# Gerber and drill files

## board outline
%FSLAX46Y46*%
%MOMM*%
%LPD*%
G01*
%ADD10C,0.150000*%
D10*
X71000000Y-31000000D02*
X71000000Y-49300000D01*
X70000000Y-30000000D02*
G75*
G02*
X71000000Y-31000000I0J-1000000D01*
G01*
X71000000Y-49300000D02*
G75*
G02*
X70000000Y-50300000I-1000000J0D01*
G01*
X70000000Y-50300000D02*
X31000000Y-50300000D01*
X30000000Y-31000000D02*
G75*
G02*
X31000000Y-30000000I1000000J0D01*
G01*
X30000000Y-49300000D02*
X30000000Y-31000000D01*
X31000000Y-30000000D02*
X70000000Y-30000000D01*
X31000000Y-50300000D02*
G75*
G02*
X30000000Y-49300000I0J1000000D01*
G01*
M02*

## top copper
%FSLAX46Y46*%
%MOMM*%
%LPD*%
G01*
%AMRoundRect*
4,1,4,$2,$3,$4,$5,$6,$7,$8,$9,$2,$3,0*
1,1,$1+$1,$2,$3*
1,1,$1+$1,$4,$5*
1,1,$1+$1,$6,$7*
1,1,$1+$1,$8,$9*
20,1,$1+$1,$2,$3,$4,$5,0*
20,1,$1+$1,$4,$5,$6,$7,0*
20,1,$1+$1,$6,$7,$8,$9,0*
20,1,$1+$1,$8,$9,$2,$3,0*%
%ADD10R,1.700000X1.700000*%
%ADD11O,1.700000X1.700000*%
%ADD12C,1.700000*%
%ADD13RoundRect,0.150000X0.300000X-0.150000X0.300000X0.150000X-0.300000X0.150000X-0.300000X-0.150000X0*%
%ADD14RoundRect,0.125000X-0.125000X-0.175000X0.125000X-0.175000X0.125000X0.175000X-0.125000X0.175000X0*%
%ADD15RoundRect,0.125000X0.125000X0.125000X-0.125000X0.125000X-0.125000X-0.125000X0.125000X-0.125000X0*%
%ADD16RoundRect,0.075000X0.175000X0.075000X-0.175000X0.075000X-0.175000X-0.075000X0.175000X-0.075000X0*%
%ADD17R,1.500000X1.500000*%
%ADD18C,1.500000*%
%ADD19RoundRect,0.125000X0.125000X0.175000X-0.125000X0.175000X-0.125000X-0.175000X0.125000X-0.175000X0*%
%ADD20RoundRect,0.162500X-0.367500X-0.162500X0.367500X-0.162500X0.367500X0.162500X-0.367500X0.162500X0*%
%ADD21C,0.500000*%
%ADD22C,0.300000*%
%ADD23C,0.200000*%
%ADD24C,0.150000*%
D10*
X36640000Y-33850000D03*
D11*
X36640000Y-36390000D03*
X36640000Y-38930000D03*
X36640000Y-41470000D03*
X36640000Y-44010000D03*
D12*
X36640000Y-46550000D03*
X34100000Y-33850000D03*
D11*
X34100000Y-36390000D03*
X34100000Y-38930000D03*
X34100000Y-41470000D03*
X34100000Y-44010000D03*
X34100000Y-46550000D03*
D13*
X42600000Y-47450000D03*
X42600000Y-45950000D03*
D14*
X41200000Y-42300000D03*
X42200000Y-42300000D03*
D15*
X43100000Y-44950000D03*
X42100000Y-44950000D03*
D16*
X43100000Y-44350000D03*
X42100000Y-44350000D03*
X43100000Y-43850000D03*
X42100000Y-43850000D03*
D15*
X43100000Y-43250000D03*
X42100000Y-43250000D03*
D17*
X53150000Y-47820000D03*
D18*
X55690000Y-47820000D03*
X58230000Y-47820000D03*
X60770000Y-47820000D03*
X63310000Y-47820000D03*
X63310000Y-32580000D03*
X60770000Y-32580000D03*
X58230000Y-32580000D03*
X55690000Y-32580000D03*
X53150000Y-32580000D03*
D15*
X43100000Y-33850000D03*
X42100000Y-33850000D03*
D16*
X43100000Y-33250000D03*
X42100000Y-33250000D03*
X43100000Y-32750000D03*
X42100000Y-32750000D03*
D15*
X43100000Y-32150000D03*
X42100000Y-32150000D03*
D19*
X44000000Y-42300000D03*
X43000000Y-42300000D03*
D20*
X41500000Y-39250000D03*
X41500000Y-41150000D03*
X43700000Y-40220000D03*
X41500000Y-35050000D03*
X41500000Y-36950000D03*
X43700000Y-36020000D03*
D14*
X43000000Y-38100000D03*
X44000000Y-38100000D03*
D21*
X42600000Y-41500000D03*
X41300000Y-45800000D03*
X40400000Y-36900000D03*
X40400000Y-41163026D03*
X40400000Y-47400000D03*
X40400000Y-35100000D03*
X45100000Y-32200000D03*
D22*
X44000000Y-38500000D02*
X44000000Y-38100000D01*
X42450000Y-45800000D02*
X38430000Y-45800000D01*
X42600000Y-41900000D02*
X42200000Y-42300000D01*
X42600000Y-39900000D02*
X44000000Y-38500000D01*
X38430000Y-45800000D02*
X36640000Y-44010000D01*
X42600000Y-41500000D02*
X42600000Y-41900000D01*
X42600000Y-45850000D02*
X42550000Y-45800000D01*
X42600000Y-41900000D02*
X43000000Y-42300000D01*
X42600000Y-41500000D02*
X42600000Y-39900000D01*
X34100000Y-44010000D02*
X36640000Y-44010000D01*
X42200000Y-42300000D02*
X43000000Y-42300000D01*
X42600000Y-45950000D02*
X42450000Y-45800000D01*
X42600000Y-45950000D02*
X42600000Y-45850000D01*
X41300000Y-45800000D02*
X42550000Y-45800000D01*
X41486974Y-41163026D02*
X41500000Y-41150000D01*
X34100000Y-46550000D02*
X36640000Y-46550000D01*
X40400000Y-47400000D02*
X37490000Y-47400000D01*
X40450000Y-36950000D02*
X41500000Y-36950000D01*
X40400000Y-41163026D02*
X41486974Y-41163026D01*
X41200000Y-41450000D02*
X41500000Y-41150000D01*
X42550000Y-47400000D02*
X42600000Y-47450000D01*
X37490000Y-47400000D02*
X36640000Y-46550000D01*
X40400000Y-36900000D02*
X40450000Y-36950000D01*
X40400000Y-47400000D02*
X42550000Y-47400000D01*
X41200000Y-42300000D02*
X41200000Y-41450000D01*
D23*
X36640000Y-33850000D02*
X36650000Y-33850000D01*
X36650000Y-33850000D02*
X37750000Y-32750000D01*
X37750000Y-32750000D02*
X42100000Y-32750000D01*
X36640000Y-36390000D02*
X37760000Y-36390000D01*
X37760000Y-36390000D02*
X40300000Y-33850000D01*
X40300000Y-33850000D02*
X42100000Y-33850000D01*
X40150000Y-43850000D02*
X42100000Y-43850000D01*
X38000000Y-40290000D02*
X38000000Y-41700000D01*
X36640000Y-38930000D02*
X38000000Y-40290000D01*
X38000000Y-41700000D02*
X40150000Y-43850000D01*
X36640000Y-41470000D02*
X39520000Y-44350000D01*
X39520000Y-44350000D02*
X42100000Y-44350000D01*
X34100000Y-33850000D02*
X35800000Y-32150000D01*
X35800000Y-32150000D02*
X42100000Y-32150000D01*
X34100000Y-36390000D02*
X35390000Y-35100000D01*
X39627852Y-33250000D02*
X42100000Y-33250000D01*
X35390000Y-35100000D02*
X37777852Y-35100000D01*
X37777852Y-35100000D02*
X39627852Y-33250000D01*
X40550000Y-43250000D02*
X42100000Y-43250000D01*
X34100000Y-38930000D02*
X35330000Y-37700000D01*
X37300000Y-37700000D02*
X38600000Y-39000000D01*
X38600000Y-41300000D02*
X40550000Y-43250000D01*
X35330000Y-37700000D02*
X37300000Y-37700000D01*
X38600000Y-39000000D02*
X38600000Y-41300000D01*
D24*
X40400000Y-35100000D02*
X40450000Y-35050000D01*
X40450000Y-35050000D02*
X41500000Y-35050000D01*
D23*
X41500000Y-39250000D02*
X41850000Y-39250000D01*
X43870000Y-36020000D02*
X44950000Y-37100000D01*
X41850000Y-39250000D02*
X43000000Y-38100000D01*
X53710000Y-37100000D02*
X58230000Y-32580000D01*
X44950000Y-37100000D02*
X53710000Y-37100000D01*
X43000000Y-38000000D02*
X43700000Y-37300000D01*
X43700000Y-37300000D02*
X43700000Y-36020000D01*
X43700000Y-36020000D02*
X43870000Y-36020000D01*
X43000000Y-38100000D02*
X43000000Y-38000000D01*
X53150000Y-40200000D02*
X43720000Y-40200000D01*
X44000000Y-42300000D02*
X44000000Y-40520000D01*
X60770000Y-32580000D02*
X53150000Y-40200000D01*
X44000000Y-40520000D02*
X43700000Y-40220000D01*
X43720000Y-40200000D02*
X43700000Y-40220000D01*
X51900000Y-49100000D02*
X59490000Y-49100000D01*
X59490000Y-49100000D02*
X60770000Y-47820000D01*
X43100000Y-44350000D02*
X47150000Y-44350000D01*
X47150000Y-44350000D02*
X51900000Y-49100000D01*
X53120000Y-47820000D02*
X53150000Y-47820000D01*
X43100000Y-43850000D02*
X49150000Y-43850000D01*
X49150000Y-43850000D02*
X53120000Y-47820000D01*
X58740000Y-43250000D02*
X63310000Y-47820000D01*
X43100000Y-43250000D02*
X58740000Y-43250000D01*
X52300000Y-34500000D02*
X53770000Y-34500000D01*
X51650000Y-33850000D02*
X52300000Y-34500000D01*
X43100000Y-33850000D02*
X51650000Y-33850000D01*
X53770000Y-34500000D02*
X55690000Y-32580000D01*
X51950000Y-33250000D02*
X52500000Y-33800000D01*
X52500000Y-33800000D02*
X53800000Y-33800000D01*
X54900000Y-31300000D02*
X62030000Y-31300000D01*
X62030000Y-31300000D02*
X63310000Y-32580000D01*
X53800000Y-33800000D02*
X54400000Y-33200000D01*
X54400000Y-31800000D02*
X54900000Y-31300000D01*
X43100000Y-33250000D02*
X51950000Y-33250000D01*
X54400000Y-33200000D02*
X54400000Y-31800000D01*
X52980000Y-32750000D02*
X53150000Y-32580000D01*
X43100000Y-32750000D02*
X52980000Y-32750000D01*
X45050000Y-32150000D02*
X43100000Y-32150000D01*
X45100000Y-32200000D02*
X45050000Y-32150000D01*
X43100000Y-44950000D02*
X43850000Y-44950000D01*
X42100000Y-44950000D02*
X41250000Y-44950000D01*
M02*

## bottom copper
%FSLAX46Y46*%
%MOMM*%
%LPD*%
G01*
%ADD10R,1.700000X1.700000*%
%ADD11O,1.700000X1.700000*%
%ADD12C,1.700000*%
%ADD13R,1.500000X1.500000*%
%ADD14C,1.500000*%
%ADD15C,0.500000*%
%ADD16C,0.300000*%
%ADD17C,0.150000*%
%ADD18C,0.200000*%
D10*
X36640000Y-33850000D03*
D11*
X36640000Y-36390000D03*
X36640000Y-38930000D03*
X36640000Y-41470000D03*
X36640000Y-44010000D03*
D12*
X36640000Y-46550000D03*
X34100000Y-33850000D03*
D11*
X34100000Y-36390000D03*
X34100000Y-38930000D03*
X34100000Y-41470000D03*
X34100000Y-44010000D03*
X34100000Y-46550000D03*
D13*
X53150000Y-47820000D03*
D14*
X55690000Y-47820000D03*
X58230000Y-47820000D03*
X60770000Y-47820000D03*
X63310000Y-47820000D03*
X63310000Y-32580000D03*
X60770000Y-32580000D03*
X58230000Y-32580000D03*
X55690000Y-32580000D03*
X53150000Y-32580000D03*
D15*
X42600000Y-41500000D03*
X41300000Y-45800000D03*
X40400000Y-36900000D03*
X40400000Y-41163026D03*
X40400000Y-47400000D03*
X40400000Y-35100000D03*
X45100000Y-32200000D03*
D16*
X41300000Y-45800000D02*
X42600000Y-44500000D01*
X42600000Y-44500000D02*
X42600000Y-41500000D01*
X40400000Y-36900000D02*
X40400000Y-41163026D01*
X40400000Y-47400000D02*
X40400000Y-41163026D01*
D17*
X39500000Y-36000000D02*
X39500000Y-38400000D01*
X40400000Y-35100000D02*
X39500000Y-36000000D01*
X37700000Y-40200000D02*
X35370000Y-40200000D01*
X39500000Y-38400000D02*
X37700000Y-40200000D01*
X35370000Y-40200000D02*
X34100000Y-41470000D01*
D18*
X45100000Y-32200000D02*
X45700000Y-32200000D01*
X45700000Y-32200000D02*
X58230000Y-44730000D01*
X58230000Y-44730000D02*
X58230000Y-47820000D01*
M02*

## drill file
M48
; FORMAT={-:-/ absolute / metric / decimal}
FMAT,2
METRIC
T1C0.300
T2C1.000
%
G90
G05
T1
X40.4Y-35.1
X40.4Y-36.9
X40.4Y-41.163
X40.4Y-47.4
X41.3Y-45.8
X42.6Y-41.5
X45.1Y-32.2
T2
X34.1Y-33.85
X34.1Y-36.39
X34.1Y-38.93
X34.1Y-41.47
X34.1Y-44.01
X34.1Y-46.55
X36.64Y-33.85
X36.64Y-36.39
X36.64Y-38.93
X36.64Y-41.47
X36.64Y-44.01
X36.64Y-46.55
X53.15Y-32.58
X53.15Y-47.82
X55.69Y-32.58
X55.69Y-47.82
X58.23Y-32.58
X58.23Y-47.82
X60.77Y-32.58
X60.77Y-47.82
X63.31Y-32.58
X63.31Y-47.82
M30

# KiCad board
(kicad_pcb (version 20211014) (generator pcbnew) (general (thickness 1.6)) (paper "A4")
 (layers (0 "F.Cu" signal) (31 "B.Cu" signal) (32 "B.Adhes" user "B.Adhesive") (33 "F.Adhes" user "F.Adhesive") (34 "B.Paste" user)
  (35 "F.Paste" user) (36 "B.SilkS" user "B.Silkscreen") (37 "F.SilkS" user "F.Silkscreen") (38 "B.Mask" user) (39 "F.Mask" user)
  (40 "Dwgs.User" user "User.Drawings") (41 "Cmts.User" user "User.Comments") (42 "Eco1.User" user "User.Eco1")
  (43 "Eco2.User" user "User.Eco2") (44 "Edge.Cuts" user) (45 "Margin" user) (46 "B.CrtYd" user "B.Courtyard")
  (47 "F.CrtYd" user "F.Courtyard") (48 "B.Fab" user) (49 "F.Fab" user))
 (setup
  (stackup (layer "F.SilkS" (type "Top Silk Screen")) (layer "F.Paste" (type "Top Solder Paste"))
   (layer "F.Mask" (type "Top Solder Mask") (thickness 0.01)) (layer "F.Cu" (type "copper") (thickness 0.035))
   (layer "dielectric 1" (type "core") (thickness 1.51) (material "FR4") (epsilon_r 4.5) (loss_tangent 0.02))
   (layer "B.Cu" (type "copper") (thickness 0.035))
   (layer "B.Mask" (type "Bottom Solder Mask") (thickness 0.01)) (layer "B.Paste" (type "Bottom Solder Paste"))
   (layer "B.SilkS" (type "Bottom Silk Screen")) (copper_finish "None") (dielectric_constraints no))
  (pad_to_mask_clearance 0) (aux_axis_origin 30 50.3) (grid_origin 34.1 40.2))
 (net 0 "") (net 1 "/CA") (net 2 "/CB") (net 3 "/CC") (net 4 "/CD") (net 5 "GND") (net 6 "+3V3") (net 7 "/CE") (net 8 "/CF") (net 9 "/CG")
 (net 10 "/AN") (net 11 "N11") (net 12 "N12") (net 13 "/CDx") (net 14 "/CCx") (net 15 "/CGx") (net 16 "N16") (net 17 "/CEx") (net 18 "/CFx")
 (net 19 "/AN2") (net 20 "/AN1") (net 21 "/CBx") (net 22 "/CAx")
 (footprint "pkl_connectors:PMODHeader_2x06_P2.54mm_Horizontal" (layer "F.Cu") (at 36.64 46.55 180)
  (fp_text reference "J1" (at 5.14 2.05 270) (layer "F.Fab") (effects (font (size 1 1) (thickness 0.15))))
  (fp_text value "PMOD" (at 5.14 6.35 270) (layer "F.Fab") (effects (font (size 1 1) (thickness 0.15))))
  (pad "1" thru_hole rect (at 0 12.7 180) (size 1.7 1.7) (drill 1) (layers *.Cu *.Mask) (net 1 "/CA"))
  (pad "2" thru_hole oval (at 0 10.16 180) (size 1.7 1.7) (drill 1) (layers *.Cu *.Mask) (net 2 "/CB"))
  (pad "3" thru_hole oval (at 0 7.62 180) (size 1.7 1.7) (drill 1) (layers *.Cu *.Mask) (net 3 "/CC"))
  (pad "4" thru_hole oval (at 0 5.08 180) (size 1.7 1.7) (drill 1) (layers *.Cu *.Mask) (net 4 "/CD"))
  (pad "5" thru_hole oval (at 0 2.54 180) (size 1.7 1.7) (drill 1) (layers *.Cu *.Mask) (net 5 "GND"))
  (pad "6" thru_hole circle (at 0 0 180) (size 1.7 1.7) (drill 1) (layers *.Cu *.Mask) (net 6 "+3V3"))
  (pad "7" thru_hole circle (at 2.54 12.7 180) (size 1.7 1.7) (drill 1) (layers *.Cu *.Mask) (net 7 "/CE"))
  (pad "8" thru_hole oval (at 2.54 10.16 180) (size 1.7 1.7) (drill 1) (layers *.Cu *.Mask) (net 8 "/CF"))
  (pad "9" thru_hole oval (at 2.54 7.62 180) (size 1.7 1.7) (drill 1) (layers *.Cu *.Mask) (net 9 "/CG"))
  (pad "10" thru_hole oval (at 2.54 5.08 180) (size 1.7 1.7) (drill 1) (layers *.Cu *.Mask) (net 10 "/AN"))
  (pad "11" thru_hole oval (at 2.54 2.54 180) (size 1.7 1.7) (drill 1) (layers *.Cu *.Mask) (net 5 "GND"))
  (pad "12" thru_hole oval (at 2.54 0 180) (size 1.7 1.7) (drill 1) (layers *.Cu *.Mask) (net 6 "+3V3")))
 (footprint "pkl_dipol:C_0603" (layer "F.Cu") (at 42.6 46.7 90)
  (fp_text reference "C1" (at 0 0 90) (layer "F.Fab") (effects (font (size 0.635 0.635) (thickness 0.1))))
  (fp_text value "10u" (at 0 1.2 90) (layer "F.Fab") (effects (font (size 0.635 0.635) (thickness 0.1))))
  (pad "1" smd roundrect locked (at -0.75 0 90) (size 0.6 0.9) (layers "F.Cu" "F.Paste" "F.Mask") (roundrect_rratio 0.25) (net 6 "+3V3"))
  (pad "2" smd roundrect locked (at 0.75 0 90) (size 0.6 0.9) (layers "F.Cu" "F.Paste" "F.Mask") (roundrect_rratio 0.25) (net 5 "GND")))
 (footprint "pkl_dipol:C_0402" (layer "F.Cu") (at 41.7 42.3)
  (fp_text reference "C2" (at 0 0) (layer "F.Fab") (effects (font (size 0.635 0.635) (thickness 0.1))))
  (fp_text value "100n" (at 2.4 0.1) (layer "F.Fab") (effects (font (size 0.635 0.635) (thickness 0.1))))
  (pad "1" smd roundrect (at -0.5 0) (size 0.5 0.6) (layers "F.Cu" "F.Paste" "F.Mask") (roundrect_rratio 0.25) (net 6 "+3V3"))
  (pad "2" smd roundrect (at 0.5 0) (size 0.5 0.6) (layers "F.Cu" "F.Paste" "F.Mask") (roundrect_rratio 0.25) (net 5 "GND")))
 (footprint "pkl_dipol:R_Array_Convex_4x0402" (layer "F.Cu") (at 42.6 44.1 180) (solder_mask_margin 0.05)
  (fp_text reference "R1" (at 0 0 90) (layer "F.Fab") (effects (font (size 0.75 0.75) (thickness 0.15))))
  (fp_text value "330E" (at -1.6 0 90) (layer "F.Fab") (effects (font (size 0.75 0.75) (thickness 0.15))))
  (pad "1" smd roundrect locked (at -0.5 -0.85 180) (size 0.5 0.5) (layers "F.Cu" "F.Paste" "F.Mask") (roundrect_rratio 0.25) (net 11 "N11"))
  (pad "2" smd roundrect locked (at 0.5 -0.85 180) (size 0.5 0.5) (layers "F.Cu" "F.Paste" "F.Mask") (roundrect_rratio 0.25) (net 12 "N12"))
  (pad "3" smd roundrect locked (at -0.5 -0.25 180) (size 0.5 0.3) (layers "F.Cu" "F.Paste" "F.Mask") (roundrect_rratio 0.25)
   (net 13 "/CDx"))
  (pad "4" smd roundrect locked (at 0.5 -0.25 180) (size 0.5 0.3) (layers "F.Cu" "F.Paste" "F.Mask") (roundrect_rratio 0.25) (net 4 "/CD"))
  (pad "5" smd roundrect locked (at -0.5 0.25 180) (size 0.5 0.3) (layers "F.Cu" "F.Paste" "F.Mask") (roundrect_rratio 0.25) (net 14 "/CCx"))
  (pad "6" smd roundrect locked (at 0.5 0.25 180) (size 0.5 0.3) (layers "F.Cu" "F.Paste" "F.Mask") (roundrect_rratio 0.25) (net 3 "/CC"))
  (pad "7" smd roundrect locked (at -0.5 0.85 180) (size 0.5 0.5) (layers "F.Cu" "F.Paste" "F.Mask") (roundrect_rratio 0.25) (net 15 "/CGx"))
  (pad "8" smd roundrect locked (at 0.5 0.85 180) (size 0.5 0.5) (layers "F.Cu" "F.Paste" "F.Mask") (roundrect_rratio 0.25) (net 9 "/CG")))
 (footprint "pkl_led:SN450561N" (layer "F.Cu") (at 53.15 47.82 90)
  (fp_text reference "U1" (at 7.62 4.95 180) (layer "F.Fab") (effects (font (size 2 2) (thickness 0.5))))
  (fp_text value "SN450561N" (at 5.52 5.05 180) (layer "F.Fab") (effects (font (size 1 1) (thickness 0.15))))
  (pad "1" thru_hole rect locked (at 0 0 90) (size 1.5 1.5) (drill 1) (layers *.Cu *.Mask) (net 14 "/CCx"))
  (pad "2" thru_hole circle locked (at 0 2.54 90) (size 1.5 1.5) (drill 1) (layers *.Cu *.Mask) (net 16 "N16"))
  (pad "3" thru_hole circle locked (at 0 5.08 90) (size 1.5 1.5) (drill 1) (layers *.Cu *.Mask) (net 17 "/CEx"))
  (pad "4" thru_hole circle locked (at 0 7.62 90) (size 1.5 1.5) (drill 1) (layers *.Cu *.Mask) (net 13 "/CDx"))
  (pad "5" thru_hole circle locked (at 0 10.16 90) (size 1.5 1.5) (drill 1) (layers *.Cu *.Mask) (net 15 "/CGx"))
  (pad "6" thru_hole circle locked (at 15.24 10.16 90) (size 1.5 1.5) (drill 1) (layers *.Cu *.Mask) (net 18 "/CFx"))
  (pad "7" thru_hole circle locked (at 15.24 7.62 90) (size 1.5 1.5) (drill 1) (layers *.Cu *.Mask) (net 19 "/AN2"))
  (pad "8" thru_hole circle locked (at 15.24 5.08 90) (size 1.5 1.5) (drill 1) (layers *.Cu *.Mask) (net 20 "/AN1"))
  (pad "9" thru_hole circle locked (at 15.24 2.54 90) (size 1.5 1.5) (drill 1) (layers *.Cu *.Mask) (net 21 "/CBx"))
  (pad "10" thru_hole circle locked (at 15.24 0 90) (size 1.5 1.5) (drill 1) (layers *.Cu *.Mask) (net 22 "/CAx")))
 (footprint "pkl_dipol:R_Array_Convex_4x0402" (layer "F.Cu") (at 42.6 33 180) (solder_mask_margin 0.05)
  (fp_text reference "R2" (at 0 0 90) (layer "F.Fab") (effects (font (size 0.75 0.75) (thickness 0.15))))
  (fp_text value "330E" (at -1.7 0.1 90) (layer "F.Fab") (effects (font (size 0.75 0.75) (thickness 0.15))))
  (pad "1" smd roundrect locked (at -0.5 -0.85 180) (size 0.5 0.5) (layers "F.Cu" "F.Paste" "F.Mask") (roundrect_rratio 0.25)
   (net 21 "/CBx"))
  (pad "2" smd roundrect locked (at 0.5 -0.85 180) (size 0.5 0.5) (layers "F.Cu" "F.Paste" "F.Mask") (roundrect_rratio 0.25) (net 2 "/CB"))
  (pad "3" smd roundrect locked (at -0.5 -0.25 180) (size 0.5 0.3) (layers "F.Cu" "F.Paste" "F.Mask") (roundrect_rratio 0.25)
   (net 18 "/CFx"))
  (pad "4" smd roundrect locked (at 0.5 -0.25 180) (size 0.5 0.3) (layers "F.Cu" "F.Paste" "F.Mask") (roundrect_rratio 0.25) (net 8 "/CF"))
  (pad "5" smd roundrect locked (at -0.5 0.25 180) (size 0.5 0.3) (layers "F.Cu" "F.Paste" "F.Mask") (roundrect_rratio 0.25) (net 22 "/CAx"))
  (pad "6" smd roundrect locked (at 0.5 0.25 180) (size 0.5 0.3) (layers "F.Cu" "F.Paste" "F.Mask") (roundrect_rratio 0.25) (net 1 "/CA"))
  (pad "7" smd roundrect locked (at -0.5 0.85 180) (size 0.5 0.5) (layers "F.Cu" "F.Paste" "F.Mask") (roundrect_rratio 0.25) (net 17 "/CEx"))
  (pad "8" smd roundrect locked (at 0.5 0.85 180) (size 0.5 0.5) (layers "F.Cu" "F.Paste" "F.Mask") (roundrect_rratio 0.25) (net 7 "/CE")))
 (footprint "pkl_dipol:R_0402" (layer "F.Cu") (at 43.5 42.3 180)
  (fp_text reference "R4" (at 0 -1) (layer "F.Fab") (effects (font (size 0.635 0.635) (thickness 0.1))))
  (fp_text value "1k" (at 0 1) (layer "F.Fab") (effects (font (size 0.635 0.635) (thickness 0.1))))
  (pad "1" smd roundrect (at -0.5 0 180) (size 0.5 0.6) (layers "F.Cu" "F.Paste" "F.Mask") (roundrect_rratio 0.25) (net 19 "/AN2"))
  (pad "2" smd roundrect (at 0.5 0 180) (size 0.5 0.6) (layers "F.Cu" "F.Paste" "F.Mask") (roundrect_rratio 0.25) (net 5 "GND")))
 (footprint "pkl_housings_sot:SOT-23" (layer "F.Cu") (at 42.6 40.2 180)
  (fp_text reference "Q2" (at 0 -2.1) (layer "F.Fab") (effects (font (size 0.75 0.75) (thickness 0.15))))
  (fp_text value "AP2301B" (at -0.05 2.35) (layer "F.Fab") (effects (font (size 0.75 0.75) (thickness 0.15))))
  (pad "1" smd roundrect locked (at 1.1 0.95) (size 1.06 0.65) (layers "F.Cu" "F.Paste" "F.Mask") (roundrect_rratio 0.25) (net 20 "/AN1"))
  (pad "2" smd roundrect locked (at 1.1 -0.95) (size 1.06 0.65) (layers "F.Cu" "F.Paste" "F.Mask") (roundrect_rratio 0.25) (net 6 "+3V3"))
  (pad "3" smd roundrect locked (at -1.1 -0.02) (size 1.06 0.65) (layers "F.Cu" "F.Paste" "F.Mask") (roundrect_rratio 0.25) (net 19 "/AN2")))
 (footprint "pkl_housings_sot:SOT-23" (layer "F.Cu") (at 42.6 36 180)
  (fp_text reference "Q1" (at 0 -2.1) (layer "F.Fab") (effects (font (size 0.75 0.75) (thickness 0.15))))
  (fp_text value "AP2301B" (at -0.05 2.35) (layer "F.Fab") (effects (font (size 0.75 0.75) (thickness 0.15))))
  (pad "1" smd roundrect locked (at 1.1 0.95) (size 1.06 0.65) (layers "F.Cu" "F.Paste" "F.Mask") (roundrect_rratio 0.25) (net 10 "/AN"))
  (pad "2" smd roundrect locked (at 1.1 -0.95) (size 1.06 0.65) (layers "F.Cu" "F.Paste" "F.Mask") (roundrect_rratio 0.25) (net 6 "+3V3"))
  (pad "3" smd roundrect locked (at -1.1 -0.02) (size 1.06 0.65) (layers "F.Cu" "F.Paste" "F.Mask") (roundrect_rratio 0.25) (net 20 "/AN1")))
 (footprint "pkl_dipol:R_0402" (layer "F.Cu") (at 43.5 38.1)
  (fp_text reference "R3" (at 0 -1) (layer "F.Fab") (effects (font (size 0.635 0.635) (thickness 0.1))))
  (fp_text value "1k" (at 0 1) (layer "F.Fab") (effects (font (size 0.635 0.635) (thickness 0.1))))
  (pad "1" smd roundrect (at -0.5 0) (size 0.5 0.6) (layers "F.Cu" "F.Paste" "F.Mask") (roundrect_rratio 0.25) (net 20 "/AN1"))
  (pad "2" smd roundrect (at 0.5 0) (size 0.5 0.6) (layers "F.Cu" "F.Paste" "F.Mask") (roundrect_rratio 0.25) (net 5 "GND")))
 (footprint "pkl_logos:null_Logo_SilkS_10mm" (layer "B.Cu") (at 49.7 40.1 90)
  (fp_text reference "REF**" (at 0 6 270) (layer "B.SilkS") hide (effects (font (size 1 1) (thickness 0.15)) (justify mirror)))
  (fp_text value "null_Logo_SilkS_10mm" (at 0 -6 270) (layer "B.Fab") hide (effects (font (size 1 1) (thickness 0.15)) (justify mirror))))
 (gr_line (start 71 31) (end 71 49.3) (layer "Edge.Cuts") (width 0.15))
 (gr_arc (start 70 30) (mid 70.707107 30.292893) (end 71 31) (layer "Edge.Cuts") (width 0.15))
 (gr_arc (start 71 49.3) (mid 70.707107 50.007107) (end 70 50.3) (layer "Edge.Cuts") (width 0.15))
 (gr_line (start 70 50.3) (end 31 50.3) (layer "Edge.Cuts") (width 0.15))
 (gr_arc (start 30 31) (mid 30.292893 30.292893) (end 31 30) (layer "Edge.Cuts") (width 0.15))
 (gr_line (start 30 49.3) (end 30 31) (layer "Edge.Cuts") (width 0.15))
 (gr_line (start 31 30) (end 70 30) (layer "Edge.Cuts") (width 0.15))
 (gr_arc (start 31 50.3) (mid 30.292893 50.007107) (end 30 49.3) (layer "Edge.Cuts") (width 0.15))
 (segment (start 44 38.5) (end 44 38.1) (width 0.3) (layer "F.Cu") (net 5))
 (segment (start 42.45 45.8) (end 38.43 45.8) (width 0.3) (layer "F.Cu") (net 5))
 (segment (start 42.6 41.9) (end 42.2 42.3) (width 0.3) (layer "F.Cu") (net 5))
 (segment (start 42.6 39.9) (end 44 38.5) (width 0.3) (layer "F.Cu") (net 5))
 (segment (start 38.43 45.8) (end 36.64 44.01) (width 0.3) (layer "F.Cu") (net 5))
 (segment (start 42.6 41.5) (end 42.6 41.9) (width 0.3) (layer "F.Cu") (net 5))
 (segment (start 42.6 45.85) (end 42.55 45.8) (width 0.3) (layer "F.Cu") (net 5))
 (segment (start 42.6 41.9) (end 43 42.3) (width 0.3) (layer "F.Cu") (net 5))
 (segment (start 42.6 41.5) (end 42.6 39.9) (width 0.3) (layer "F.Cu") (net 5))
 (segment (start 34.1 44.01) (end 36.64 44.01) (width 0.3) (layer "F.Cu") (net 5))
 (segment (start 42.2 42.3) (end 43 42.3) (width 0.3) (layer "F.Cu") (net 5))
 (segment (start 42.6 45.95) (end 42.45 45.8) (width 0.3) (layer "F.Cu") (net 5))
 (segment (start 42.6 45.95) (end 42.6 45.85) (width 0.3) (layer "F.Cu") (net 5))
 (segment (start 41.3 45.8) (end 42.55 45.8) (width 0.3) (layer "F.Cu") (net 5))
 (via (at 42.6 41.5) (size 0.5) (drill 0.3) (layers "F.Cu" "B.Cu") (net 5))
 (via (at 41.3 45.8) (size 0.5) (drill 0.3) (layers "F.Cu" "B.Cu") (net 5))
 (segment (start 41.3 45.8) (end 42.6 44.5) (width 0.3) (layer "B.Cu") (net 5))
 (segment (start 42.6 44.5) (end 42.6 41.5) (width 0.3) (layer "B.Cu") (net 5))
 (segment (start 41.486974 41.163026) (end 41.5 41.15) (width 0.3) (layer "F.Cu") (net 6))
 (segment (start 34.1 46.55) (end 36.64 46.55) (width 0.3) (layer "F.Cu") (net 6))
 (segment (start 40.4 47.4) (end 37.49 47.4) (width 0.3) (layer "F.Cu") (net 6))
 (segment (start 40.45 36.95) (end 41.5 36.95) (width 0.3) (layer "F.Cu") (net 6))
 (segment (start 40.4 41.163026) (end 41.486974 41.163026) (width 0.3) (layer "F.Cu") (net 6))
 (segment (start 41.2 41.45) (end 41.5 41.15) (width 0.3) (layer "F.Cu") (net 6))
 (segment (start 42.55 47.4) (end 42.6 47.45) (width 0.3) (layer "F.Cu") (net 6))
 (segment (start 37.49 47.4) (end 36.64 46.55) (width 0.3) (layer "F.Cu") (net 6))
 (segment (start 40.4 36.9) (end 40.45 36.95) (width 0.3) (layer "F.Cu") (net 6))
 (segment (start 40.4 47.4) (end 42.55 47.4) (width 0.3) (layer "F.Cu") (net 6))
 (segment (start 41.2 42.3) (end 41.2 41.45) (width 0.3) (layer "F.Cu") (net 6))
 (via (at 40.4 36.9) (size 0.5) (drill 0.3) (layers "F.Cu" "B.Cu") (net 6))
 (via (at 40.4 41.163026) (size 0.5) (drill 0.3) (layers "F.Cu" "B.Cu") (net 6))
 (via (at 40.4 47.4) (size 0.5) (drill 0.3) (layers "F.Cu" "B.Cu") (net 6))
 (segment (start 40.4 36.9) (end 40.4 41.163026) (width 0.3) (layer "B.Cu") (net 6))
 (segment (start 40.4 47.4) (end 40.4 41.163026) (width 0.3) (layer "B.Cu") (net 6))
 (segment (start 36.64 33.85) (end 36.65 33.85) (width 0.2) (layer "F.Cu") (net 1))
 (segment (start 36.65 33.85) (end 37.75 32.75) (width 0.2) (layer "F.Cu") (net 1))
 (segment (start 37.75 32.75) (end 42.1 32.75) (width 0.2) (layer "F.Cu") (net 1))
 (segment (start 36.64 36.39) (end 37.76 36.39) (width 0.2) (layer "F.Cu") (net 2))
 (segment (start 37.76 36.39) (end 40.3 33.85) (width 0.2) (layer "F.Cu") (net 2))
 (segment (start 40.3 33.85) (end 42.1 33.85) (width 0.2) (layer "F.Cu") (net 2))
 (segment (start 40.15 43.85) (end 42.1 43.85) (width 0.2) (layer "F.Cu") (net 3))
 (segment (start 38 40.29) (end 38 41.7) (width 0.2) (layer "F.Cu") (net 3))
 (segment (start 36.64 38.93) (end 38 40.29) (width 0.2) (layer "F.Cu") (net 3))
 (segment (start 38 41.7) (end 40.15 43.85) (width 0.2) (layer "F.Cu") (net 3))
 (segment (start 36.64 41.47) (end 39.52 44.35) (width 0.2) (layer "F.Cu") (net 4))
 (segment (start 39.52 44.35) (end 42.1 44.35) (width 0.2) (layer "F.Cu") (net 4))
 (segment (start 34.1 33.85) (end 35.8 32.15) (width 0.2) (layer "F.Cu") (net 7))
 (segment (start 35.8 32.15) (end 42.1 32.15) (width 0.2) (layer "F.Cu") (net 7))
 (segment (start 34.1 36.39) (end 35.39 35.1) (width 0.2) (layer "F.Cu") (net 8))
 (segment (start 39.627852 33.25) (end 42.1 33.25) (width 0.2) (layer "F.Cu") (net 8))
 (segment (start 35.39 35.1) (end 37.777852 35.1) (width 0.2) (layer "F.Cu") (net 8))
 (segment (start 37.777852 35.1) (end 39.627852 33.25) (width 0.2) (layer "F.Cu") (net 8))
 (segment (start 40.55 43.25) (end 42.1 43.25) (width 0.2) (layer "F.Cu") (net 9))
 (segment (start 34.1 38.93) (end 35.33 37.7) (width 0.2) (layer "F.Cu") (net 9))
 (segment (start 37.3 37.7) (end 38.6 39) (width 0.2) (layer "F.Cu") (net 9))
 (segment (start 38.6 41.3) (end 40.55 43.25) (width 0.2) (layer "F.Cu") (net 9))
 (segment (start 35.33 37.7) (end 37.3 37.7) (width 0.2) (layer "F.Cu") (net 9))
 (segment (start 38.6 39) (end 38.6 41.3) (width 0.2) (layer "F.Cu") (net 9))
 (segment (start 40.4 35.1) (end 40.45 35.05) (width 0.15) (layer "F.Cu") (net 10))
 (segment (start 40.45 35.05) (end 41.5 35.05) (width 0.15) (layer "F.Cu") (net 10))
 (via (at 40.4 35.1) (size 0.5) (drill 0.3) (layers "F.Cu" "B.Cu") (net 10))
 (segment (start 39.5 36) (end 39.5 38.4) (width 0.15) (layer "B.Cu") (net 10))
 (segment (start 40.4 35.1) (end 39.5 36) (width 0.15) (layer "B.Cu") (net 10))
 (segment (start 37.7 40.2) (end 35.37 40.2) (width 0.15) (layer "B.Cu") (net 10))
 (segment (start 39.5 38.4) (end 37.7 40.2) (width 0.15) (layer "B.Cu") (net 10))
 (segment (start 35.37 40.2) (end 34.1 41.47) (width 0.15) (layer "B.Cu") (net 10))
 (segment (start 41.5 39.25) (end 41.85 39.25) (width 0.2) (layer "F.Cu") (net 20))
 (segment (start 43.87 36.02) (end 44.95 37.1) (width 0.2) (layer "F.Cu") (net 20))
 (segment (start 41.85 39.25) (end 43 38.1) (width 0.2) (layer "F.Cu") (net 20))
 (segment (start 53.71 37.1) (end 58.23 32.58) (width 0.2) (layer "F.Cu") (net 20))
 (segment (start 44.95 37.1) (end 53.71 37.1) (width 0.2) (layer "F.Cu") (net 20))
 (segment (start 43 38) (end 43.7 37.3) (width 0.2) (layer "F.Cu") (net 20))
 (segment (start 43.7 37.3) (end 43.7 36.02) (width 0.2) (layer "F.Cu") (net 20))
 (segment (start 43.7 36.02) (end 43.87 36.02) (width 0.2) (layer "F.Cu") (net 20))
 (segment (start 43 38.1) (end 43 38) (width 0.2) (layer "F.Cu") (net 20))
 (segment (start 53.15 40.2) (end 43.72 40.2) (width 0.2) (layer "F.Cu") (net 19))
 (segment (start 44 42.3) (end 44 40.52) (width 0.2) (layer "F.Cu") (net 19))
 (segment (start 60.77 32.58) (end 53.15 40.2) (width 0.2) (layer "F.Cu") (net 19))
 (segment (start 44 40.52) (end 43.7 40.22) (width 0.2) (layer "F.Cu") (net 19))
 (segment (start 43.72 40.2) (end 43.7 40.22) (width 0.2) (layer "F.Cu") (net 19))
 (segment (start 51.9 49.1) (end 59.49 49.1) (width 0.2) (layer "F.Cu") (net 13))
 (segment (start 59.49 49.1) (end 60.77 47.82) (width 0.2) (layer "F.Cu") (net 13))
 (segment (start 43.1 44.35) (end 47.15 44.35) (width 0.2) (layer "F.Cu") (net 13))
 (segment (start 47.15 44.35) (end 51.9 49.1) (width 0.2) (layer "F.Cu") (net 13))
 (segment (start 53.12 47.82) (end 53.15 47.82) (width 0.2) (layer "F.Cu") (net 14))
 (segment (start 43.1 43.85) (end 49.15 43.85) (width 0.2) (layer "F.Cu") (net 14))
 (segment (start 49.15 43.85) (end 53.12 47.82) (width 0.2) (layer "F.Cu") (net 14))
 (segment (start 58.74 43.25) (end 63.31 47.82) (width 0.2) (layer "F.Cu") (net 15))
 (segment (start 43.1 43.25) (end 58.74 43.25) (width 0.2) (layer "F.Cu") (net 15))
 (segment (start 52.3 34.5) (end 53.77 34.5) (width 0.2) (layer "F.Cu") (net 21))
 (segment (start 51.65 33.85) (end 52.3 34.5) (width 0.2) (layer "F.Cu") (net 21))
 (segment (start 43.1 33.85) (end 51.65 33.85) (width 0.2) (layer "F.Cu") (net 21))
 (segment (start 53.77 34.5) (end 55.69 32.58) (width 0.2) (layer "F.Cu") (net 21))
 (segment (start 51.95 33.25) (end 52.5 33.8) (width 0.2) (layer "F.Cu") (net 18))
 (segment (start 52.5 33.8) (end 53.8 33.8) (width 0.2) (layer "F.Cu") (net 18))
 (segment (start 54.9 31.3) (end 62.03 31.3) (width 0.2) (layer "F.Cu") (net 18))
 (segment (start 62.03 31.3) (end 63.31 32.58) (width 0.2) (layer "F.Cu") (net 18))
 (segment (start 53.8 33.8) (end 54.4 33.2) (width 0.2) (layer "F.Cu") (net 18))
 (segment (start 54.4 31.8) (end 54.9 31.3) (width 0.2) (layer "F.Cu") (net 18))
 (segment (start 43.1 33.25) (end 51.95 33.25) (width 0.2) (layer "F.Cu") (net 18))
 (segment (start 54.4 33.2) (end 54.4 31.8) (width 0.2) (layer "F.Cu") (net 18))
 (segment (start 52.98 32.75) (end 53.15 32.58) (width 0.2) (layer "F.Cu") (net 22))
 (segment (start 43.1 32.75) (end 52.98 32.75) (width 0.2) (layer "F.Cu") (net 22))
 (segment (start 45.05 32.15) (end 43.1 32.15) (width 0.2) (layer "F.Cu") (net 17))
 (segment (start 45.1 32.2) (end 45.05 32.15) (width 0.2) (layer "F.Cu") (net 17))
 (via (at 45.1 32.2) (size 0.5) (drill 0.3) (layers "F.Cu" "B.Cu") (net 17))
 (segment (start 45.1 32.2) (end 45.7 32.2) (width 0.2) (layer "B.Cu") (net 17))
 (segment (start 45.7 32.2) (end 58.23 44.73) (width 0.2) (layer "B.Cu") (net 17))
 (segment (start 58.23 44.73) (end 58.23 47.82) (width 0.2) (layer "B.Cu") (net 17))
 (segment (start 43.1 44.95) (end 43.85 44.95) (width 0.2) (layer "F.Cu") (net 11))
 (segment (start 42.1 44.95) (end 41.25 44.95) (width 0.2) (layer "F.Cu") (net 12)))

